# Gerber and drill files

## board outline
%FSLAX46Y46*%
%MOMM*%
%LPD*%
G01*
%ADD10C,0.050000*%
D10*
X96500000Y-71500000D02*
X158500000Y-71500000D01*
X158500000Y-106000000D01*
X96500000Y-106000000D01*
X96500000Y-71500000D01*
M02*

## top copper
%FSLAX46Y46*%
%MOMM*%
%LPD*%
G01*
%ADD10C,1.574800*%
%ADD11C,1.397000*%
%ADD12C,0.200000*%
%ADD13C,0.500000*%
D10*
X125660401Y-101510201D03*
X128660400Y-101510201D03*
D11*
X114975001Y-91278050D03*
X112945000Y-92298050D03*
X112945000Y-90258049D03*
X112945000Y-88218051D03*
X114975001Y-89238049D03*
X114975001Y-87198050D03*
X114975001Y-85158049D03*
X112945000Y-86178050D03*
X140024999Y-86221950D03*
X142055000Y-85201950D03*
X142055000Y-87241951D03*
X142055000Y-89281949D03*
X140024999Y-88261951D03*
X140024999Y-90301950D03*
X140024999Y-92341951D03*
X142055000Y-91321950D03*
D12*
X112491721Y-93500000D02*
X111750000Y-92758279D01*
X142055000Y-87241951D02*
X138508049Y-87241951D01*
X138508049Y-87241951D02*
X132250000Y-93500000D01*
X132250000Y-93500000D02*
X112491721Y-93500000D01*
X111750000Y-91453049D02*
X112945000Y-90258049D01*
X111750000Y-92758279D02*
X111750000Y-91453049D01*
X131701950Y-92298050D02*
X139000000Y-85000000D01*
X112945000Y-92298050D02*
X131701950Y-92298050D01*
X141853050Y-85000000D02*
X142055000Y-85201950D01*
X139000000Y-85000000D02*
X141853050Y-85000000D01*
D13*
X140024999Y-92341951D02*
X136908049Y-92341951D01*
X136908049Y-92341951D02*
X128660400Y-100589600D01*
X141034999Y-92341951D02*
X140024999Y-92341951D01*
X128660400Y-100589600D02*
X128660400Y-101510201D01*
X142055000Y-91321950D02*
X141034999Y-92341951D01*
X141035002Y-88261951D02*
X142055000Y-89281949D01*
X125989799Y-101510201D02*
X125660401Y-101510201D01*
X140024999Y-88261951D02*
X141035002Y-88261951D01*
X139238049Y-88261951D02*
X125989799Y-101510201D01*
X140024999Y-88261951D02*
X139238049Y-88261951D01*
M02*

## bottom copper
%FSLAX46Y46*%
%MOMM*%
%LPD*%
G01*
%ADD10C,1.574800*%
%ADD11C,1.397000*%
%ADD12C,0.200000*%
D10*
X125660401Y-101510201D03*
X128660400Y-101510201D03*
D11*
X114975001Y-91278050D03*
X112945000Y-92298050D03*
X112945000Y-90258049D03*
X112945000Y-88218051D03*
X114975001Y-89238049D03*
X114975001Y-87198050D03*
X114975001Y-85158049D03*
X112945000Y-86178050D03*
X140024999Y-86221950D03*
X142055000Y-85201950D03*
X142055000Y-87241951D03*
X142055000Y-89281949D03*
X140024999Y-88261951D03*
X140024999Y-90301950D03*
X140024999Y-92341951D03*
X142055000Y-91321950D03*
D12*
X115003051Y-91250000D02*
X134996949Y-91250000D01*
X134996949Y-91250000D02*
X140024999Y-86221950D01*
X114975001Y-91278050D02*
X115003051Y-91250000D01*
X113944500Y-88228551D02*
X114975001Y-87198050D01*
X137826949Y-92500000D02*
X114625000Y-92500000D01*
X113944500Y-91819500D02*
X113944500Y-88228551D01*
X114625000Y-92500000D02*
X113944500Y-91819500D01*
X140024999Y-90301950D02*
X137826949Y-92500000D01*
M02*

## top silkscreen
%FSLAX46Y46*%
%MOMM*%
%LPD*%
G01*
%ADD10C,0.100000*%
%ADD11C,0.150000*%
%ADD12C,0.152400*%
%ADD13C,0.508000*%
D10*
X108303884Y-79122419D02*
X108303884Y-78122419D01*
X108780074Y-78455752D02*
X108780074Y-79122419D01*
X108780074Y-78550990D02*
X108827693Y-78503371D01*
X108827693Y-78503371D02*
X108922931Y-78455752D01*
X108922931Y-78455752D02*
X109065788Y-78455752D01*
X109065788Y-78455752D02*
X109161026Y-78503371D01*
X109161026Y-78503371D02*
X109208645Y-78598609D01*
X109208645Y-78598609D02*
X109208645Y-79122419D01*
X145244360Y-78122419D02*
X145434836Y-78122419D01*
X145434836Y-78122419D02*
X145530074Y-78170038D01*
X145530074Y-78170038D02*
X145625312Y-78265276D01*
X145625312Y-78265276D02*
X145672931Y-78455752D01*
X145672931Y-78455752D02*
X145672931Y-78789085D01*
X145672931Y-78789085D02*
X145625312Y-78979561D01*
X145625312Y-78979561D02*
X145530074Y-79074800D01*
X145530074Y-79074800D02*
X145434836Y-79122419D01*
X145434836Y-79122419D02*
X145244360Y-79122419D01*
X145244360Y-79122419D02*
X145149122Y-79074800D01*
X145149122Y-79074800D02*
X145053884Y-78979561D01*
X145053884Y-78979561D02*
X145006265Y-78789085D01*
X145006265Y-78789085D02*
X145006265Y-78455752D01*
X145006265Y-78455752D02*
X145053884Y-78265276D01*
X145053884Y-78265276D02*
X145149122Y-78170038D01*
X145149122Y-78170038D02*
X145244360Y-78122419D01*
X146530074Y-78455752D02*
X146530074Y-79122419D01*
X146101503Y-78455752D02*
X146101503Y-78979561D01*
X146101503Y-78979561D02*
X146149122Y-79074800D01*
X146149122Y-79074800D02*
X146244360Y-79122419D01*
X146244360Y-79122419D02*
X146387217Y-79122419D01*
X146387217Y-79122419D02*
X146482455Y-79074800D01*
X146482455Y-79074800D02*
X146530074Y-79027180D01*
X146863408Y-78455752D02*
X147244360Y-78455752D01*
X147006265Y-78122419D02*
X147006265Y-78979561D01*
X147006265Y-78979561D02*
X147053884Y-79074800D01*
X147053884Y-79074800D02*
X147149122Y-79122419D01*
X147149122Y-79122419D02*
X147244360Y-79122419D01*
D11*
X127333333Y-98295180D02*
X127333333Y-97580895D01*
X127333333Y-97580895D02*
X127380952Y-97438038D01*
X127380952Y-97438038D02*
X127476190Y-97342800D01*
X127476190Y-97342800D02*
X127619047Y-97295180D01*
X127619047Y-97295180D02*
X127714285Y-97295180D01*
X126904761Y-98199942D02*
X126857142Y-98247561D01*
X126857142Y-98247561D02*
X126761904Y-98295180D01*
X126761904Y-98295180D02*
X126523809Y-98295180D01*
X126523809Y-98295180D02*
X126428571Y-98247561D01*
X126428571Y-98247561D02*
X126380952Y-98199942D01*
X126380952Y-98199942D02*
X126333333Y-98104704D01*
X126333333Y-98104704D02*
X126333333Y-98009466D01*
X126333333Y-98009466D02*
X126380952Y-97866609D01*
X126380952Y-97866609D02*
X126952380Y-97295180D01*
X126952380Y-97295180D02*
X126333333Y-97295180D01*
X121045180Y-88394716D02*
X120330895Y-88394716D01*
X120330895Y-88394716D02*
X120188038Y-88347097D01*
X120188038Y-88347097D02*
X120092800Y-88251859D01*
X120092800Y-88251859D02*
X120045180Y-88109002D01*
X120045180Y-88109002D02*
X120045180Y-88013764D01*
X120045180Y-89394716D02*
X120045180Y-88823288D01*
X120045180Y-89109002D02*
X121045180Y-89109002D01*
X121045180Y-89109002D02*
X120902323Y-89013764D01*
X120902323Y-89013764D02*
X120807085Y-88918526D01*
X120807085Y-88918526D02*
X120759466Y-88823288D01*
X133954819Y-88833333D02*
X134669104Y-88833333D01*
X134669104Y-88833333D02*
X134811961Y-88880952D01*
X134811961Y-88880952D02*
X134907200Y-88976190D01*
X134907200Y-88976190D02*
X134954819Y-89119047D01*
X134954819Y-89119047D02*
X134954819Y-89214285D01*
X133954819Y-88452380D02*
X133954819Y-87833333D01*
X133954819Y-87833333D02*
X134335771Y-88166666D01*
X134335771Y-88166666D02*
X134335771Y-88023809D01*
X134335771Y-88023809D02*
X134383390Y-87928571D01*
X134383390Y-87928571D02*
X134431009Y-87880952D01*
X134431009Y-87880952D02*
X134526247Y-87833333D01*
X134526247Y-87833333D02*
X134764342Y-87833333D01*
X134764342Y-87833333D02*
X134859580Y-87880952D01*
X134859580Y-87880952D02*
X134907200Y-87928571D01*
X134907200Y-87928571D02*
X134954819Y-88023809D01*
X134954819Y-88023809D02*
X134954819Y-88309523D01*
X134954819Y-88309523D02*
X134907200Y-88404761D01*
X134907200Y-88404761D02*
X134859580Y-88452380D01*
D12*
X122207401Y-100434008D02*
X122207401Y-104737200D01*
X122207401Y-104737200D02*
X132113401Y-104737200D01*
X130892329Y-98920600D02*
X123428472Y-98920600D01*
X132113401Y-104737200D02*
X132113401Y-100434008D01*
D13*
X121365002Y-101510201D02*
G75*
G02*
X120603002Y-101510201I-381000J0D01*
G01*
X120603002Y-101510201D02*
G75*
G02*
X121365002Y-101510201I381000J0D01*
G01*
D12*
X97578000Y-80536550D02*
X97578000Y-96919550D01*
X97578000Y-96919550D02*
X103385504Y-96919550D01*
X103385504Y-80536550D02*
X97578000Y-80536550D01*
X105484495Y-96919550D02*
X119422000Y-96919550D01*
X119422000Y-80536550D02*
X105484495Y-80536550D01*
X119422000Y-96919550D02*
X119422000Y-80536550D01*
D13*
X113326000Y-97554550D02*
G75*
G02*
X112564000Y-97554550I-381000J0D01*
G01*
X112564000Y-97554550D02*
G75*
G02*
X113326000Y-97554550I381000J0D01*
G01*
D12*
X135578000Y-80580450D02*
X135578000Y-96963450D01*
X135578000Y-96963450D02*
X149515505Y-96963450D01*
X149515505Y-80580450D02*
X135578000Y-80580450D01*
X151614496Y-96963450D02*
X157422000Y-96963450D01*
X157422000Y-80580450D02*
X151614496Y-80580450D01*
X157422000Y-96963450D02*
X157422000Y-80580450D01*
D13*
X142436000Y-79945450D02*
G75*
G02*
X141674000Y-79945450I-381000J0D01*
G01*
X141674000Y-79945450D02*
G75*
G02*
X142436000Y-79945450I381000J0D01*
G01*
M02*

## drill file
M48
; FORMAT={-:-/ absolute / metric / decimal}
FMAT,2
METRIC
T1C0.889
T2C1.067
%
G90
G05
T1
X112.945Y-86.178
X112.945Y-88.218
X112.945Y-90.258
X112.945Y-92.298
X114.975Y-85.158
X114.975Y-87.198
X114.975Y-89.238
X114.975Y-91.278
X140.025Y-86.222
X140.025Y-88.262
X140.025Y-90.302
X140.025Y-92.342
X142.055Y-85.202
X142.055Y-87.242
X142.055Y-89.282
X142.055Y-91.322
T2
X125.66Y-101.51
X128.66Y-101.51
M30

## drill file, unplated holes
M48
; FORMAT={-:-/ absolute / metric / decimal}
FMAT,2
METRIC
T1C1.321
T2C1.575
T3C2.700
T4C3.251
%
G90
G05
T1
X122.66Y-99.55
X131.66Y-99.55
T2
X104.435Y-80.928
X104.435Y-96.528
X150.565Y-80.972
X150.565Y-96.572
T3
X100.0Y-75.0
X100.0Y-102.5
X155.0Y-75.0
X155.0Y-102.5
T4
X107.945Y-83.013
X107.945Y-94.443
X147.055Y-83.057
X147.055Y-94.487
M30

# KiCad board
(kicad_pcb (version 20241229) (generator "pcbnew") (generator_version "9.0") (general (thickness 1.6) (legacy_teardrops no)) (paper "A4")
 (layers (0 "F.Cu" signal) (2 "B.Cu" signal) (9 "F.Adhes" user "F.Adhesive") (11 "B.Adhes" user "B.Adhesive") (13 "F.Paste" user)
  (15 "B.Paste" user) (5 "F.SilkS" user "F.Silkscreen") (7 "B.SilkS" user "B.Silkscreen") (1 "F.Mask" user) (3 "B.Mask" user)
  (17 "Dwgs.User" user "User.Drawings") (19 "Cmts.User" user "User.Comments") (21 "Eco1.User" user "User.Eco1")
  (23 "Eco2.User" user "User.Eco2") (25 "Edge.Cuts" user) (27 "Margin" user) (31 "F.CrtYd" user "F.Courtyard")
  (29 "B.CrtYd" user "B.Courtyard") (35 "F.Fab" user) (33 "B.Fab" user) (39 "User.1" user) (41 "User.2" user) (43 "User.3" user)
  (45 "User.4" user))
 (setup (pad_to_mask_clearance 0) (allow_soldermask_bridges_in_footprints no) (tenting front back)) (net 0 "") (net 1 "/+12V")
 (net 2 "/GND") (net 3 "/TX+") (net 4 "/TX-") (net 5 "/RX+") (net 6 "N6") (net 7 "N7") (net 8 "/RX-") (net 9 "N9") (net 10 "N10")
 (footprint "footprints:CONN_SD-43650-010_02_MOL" (layer "F.Cu") (at 125.660401 101.510201 180)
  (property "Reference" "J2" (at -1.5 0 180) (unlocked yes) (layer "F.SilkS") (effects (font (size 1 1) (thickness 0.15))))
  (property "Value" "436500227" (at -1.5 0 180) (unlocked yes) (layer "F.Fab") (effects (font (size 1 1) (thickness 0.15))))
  (fp_line (start 3.453 1.076193) (end 3.453 -3.226999) (stroke (width 0.1524) (type solid)) (layer "F.SilkS"))
  (fp_line (start 3.453 -3.226999) (end -6.453 -3.226999) (stroke (width 0.1524) (type solid)) (layer "F.SilkS"))
  (fp_line (start -5.231928 2.589601) (end 2.231929 2.589601) (stroke (width 0.1524) (type solid)) (layer "F.SilkS"))
  (fp_line (start -6.453 -3.226999) (end -6.453 1.076193) (stroke (width 0.1524) (type solid)) (layer "F.SilkS"))
  (fp_circle (center 4.676399 0) (end 5.057399 0) (stroke (width 0.508) (type solid)) (fill no) (layer "F.SilkS"))
  (pad "" np_thru_hole circle (at -5.999998 1.960001 180) (size 1.3208 1.3208) (drill 1.3208) (layers "*.Cu" "*.Mask"))
  (pad "" np_thru_hole circle (at 2.999999 1.960001 180) (size 1.3208 1.3208) (drill 1.3208) (layers "*.Cu" "*.Mask"))
  (pad "1" thru_hole circle (at 0 0 180) (size 1.5748 1.5748) (drill 1.0668) (layers "*.Cu" "*.Mask") (remove_unused_layers no)
   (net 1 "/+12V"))
  (pad "2" thru_hole circle (at -2.999999 0 180) (size 1.5748 1.5748) (drill 1.0668) (layers "*.Cu" "*.Mask") (remove_unused_layers no)
   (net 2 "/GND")))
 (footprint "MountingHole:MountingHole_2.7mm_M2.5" (layer "F.Cu") (at 155 102.5)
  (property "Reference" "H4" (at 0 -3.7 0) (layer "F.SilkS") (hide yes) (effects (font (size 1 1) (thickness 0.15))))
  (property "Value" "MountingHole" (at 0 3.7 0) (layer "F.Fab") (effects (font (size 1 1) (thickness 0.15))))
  (pad "" np_thru_hole circle (at 0 0) (size 2.7 2.7) (drill 2.7) (layers "*.Cu" "*.Mask")))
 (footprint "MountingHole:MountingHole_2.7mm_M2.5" (layer "F.Cu") (at 155 75)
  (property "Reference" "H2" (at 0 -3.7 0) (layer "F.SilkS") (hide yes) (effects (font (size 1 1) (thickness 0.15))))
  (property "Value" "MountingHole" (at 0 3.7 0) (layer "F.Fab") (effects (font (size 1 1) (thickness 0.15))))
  (pad "" np_thru_hole circle (at 0 0) (size 2.7 2.7) (drill 2.7) (layers "*.Cu" "*.Mask")))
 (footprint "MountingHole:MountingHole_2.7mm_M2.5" (layer "F.Cu") (at 100 75)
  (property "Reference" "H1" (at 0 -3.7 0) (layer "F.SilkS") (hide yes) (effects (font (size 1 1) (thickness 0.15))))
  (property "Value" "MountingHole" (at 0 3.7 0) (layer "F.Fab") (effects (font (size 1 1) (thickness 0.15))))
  (pad "" np_thru_hole circle (at 0 0) (size 2.7 2.7) (drill 2.7) (layers "*.Cu" "*.Mask")))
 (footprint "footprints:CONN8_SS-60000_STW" (layer "F.Cu") (at 112.945 92.29805 -90)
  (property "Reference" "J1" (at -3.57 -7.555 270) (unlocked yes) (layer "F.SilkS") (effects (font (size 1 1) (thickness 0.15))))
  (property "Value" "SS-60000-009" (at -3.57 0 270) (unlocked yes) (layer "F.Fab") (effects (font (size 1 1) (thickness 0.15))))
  (fp_line (start -11.7615 15.367) (end 4.6215 15.367) (stroke (width 0.1524) (type solid)) (layer "F.SilkS"))
  (fp_line (start 4.6215 15.367) (end 4.6215 9.559496) (stroke (width 0.1524) (type solid)) (layer "F.SilkS"))
  (fp_line (start -11.7615 9.559496) (end -11.7615 15.367) (stroke (width 0.1524) (type solid)) (layer "F.SilkS"))
  (fp_line (start 4.6215 7.460505) (end 4.6215 -6.477) (stroke (width 0.1524) (type solid)) (layer "F.SilkS"))
  (fp_line (start -11.7615 -6.477) (end -11.7615 7.460505) (stroke (width 0.1524) (type solid)) (layer "F.SilkS"))
  (fp_line (start 4.6215 -6.477) (end -11.7615 -6.477) (stroke (width 0.1524) (type solid)) (layer "F.SilkS"))
  (fp_circle (center 5.2565 0) (end 5.6375 0) (stroke (width 0.508) (type solid)) (fill no) (layer "F.SilkS"))
  (pad "" np_thru_hole circle (at -11.37 8.510001 270) (size 1.5748 1.5748) (drill 1.5748) (layers))
  (pad "" np_thru_hole circle (at -9.285 5 270) (size 3.2512 3.2512) (drill 3.2512) (layers "*.Cu" "*.Mask"))
  (pad "" np_thru_hole circle (at 2.145 5 270) (size 3.2512 3.2512) (drill 3.2512) (layers "*.Cu" "*.Mask"))
  (pad "" np_thru_hole circle (at 4.229999 8.510001 270) (size 1.5748 1.5748) (drill 1.5748) (layers))
  (pad "1" thru_hole circle (at -1.02 -2.030001 270) (size 1.397 1.397) (drill 0.889) (layers "*.Cu" "*.Mask") (remove_unused_layers no)
   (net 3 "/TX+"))
  (pad "2" thru_hole circle (at 0 0 270) (size 1.397 1.397) (drill 0.889) (layers "*.Cu" "*.Mask") (remove_unused_layers no) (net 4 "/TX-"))
  (pad "3" thru_hole circle (at -2.040001 0 270) (size 1.397 1.397) (drill 0.889) (layers "*.Cu" "*.Mask") (remove_unused_layers no)
   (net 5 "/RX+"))
  (pad "4" thru_hole circle (at -4.079999 0 270) (size 1.397 1.397) (drill 0.889) (layers "*.Cu" "*.Mask") (remove_unused_layers no)
   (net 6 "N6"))
  (pad "5" thru_hole circle (at -3.060001 -2.030001 270) (size 1.397 1.397) (drill 0.889) (layers "*.Cu" "*.Mask") (remove_unused_layers no)
   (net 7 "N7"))
  (pad "6" thru_hole circle (at -5.1 -2.030001 270) (size 1.397 1.397) (drill 0.889) (layers "*.Cu" "*.Mask") (remove_unused_layers no)
   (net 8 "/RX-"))
  (pad "7" thru_hole circle (at -7.140001 -2.030001 270) (size 1.397 1.397) (drill 0.889) (layers "*.Cu" "*.Mask") (remove_unused_layers no)
   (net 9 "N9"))
  (pad "8" thru_hole circle (at -6.12 0 270) (size 1.397 1.397) (drill 0.889) (layers "*.Cu" "*.Mask") (remove_unused_layers no)
   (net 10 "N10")))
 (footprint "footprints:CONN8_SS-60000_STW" (layer "F.Cu") (at 142.055 85.20195 90)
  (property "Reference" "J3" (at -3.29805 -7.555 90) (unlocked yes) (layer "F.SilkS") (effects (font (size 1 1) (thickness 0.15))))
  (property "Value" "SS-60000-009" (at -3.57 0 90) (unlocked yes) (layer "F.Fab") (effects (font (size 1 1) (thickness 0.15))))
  (fp_line (start 4.6215 -6.477) (end -11.7615 -6.477) (stroke (width 0.1524) (type solid)) (layer "F.SilkS"))
  (fp_line (start -11.7615 -6.477) (end -11.7615 7.460505) (stroke (width 0.1524) (type solid)) (layer "F.SilkS"))
  (fp_line (start 4.6215 7.460505) (end 4.6215 -6.477) (stroke (width 0.1524) (type solid)) (layer "F.SilkS"))
  (fp_line (start -11.7615 9.559496) (end -11.7615 15.367) (stroke (width 0.1524) (type solid)) (layer "F.SilkS"))
  (fp_line (start 4.6215 15.367) (end 4.6215 9.559496) (stroke (width 0.1524) (type solid)) (layer "F.SilkS"))
  (fp_line (start -11.7615 15.367) (end 4.6215 15.367) (stroke (width 0.1524) (type solid)) (layer "F.SilkS"))
  (fp_circle (center 5.2565 0) (end 5.6375 0) (stroke (width 0.508) (type solid)) (fill no) (layer "F.SilkS"))
  (pad "" np_thru_hole circle (at -11.37 8.510001 90) (size 1.5748 1.5748) (drill 1.5748) (layers))
  (pad "" np_thru_hole circle (at -9.285 5 90) (size 3.2512 3.2512) (drill 3.2512) (layers "*.Cu" "*.Mask"))
  (pad "" np_thru_hole circle (at 2.145 5 90) (size 3.2512 3.2512) (drill 3.2512) (layers "*.Cu" "*.Mask"))
  (pad "" np_thru_hole circle (at 4.229999 8.510001 90) (size 1.5748 1.5748) (drill 1.5748) (layers))
  (pad "1" thru_hole circle (at -1.02 -2.030001 90) (size 1.397 1.397) (drill 0.889) (layers "*.Cu" "*.Mask") (remove_unused_layers no)
   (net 3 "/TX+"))
  (pad "2" thru_hole circle (at 0 0 90) (size 1.397 1.397) (drill 0.889) (layers "*.Cu" "*.Mask") (remove_unused_layers no) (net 4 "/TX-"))
  (pad "3" thru_hole circle (at -2.040001 0 90) (size 1.397 1.397) (drill 0.889) (layers "*.Cu" "*.Mask") (remove_unused_layers no)
   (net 5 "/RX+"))
  (pad "4" thru_hole circle (at -4.079999 0 90) (size 1.397 1.397) (drill 0.889) (layers "*.Cu" "*.Mask") (remove_unused_layers no)
   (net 1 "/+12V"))
  (pad "5" thru_hole circle (at -3.060001 -2.030001 90) (size 1.397 1.397) (drill 0.889) (layers "*.Cu" "*.Mask") (remove_unused_layers no)
   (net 1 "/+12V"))
  (pad "6" thru_hole circle (at -5.1 -2.030001 90) (size 1.397 1.397) (drill 0.889) (layers "*.Cu" "*.Mask") (remove_unused_layers no)
   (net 8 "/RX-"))
  (pad "7" thru_hole circle (at -7.140001 -2.030001 90) (size 1.397 1.397) (drill 0.889) (layers "*.Cu" "*.Mask") (remove_unused_layers no)
   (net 2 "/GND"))
  (pad "8" thru_hole circle (at -6.12 0 90) (size 1.397 1.397) (drill 0.889) (layers "*.Cu" "*.Mask") (remove_unused_layers no)
   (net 2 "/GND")))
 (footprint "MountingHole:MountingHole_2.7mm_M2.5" (layer "F.Cu") (at 100 102.5)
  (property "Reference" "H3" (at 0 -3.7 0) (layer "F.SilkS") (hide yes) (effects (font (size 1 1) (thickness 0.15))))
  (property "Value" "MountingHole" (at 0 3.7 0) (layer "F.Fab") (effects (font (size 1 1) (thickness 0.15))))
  (pad "" np_thru_hole circle (at 0 0) (size 2.7 2.7) (drill 2.7) (layers "*.Cu" "*.Mask")))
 (gr_rect (start 96.5 71.5) (end 158.5 106) (stroke (width 0.05) (type default)) (fill no) (layer "Edge.Cuts"))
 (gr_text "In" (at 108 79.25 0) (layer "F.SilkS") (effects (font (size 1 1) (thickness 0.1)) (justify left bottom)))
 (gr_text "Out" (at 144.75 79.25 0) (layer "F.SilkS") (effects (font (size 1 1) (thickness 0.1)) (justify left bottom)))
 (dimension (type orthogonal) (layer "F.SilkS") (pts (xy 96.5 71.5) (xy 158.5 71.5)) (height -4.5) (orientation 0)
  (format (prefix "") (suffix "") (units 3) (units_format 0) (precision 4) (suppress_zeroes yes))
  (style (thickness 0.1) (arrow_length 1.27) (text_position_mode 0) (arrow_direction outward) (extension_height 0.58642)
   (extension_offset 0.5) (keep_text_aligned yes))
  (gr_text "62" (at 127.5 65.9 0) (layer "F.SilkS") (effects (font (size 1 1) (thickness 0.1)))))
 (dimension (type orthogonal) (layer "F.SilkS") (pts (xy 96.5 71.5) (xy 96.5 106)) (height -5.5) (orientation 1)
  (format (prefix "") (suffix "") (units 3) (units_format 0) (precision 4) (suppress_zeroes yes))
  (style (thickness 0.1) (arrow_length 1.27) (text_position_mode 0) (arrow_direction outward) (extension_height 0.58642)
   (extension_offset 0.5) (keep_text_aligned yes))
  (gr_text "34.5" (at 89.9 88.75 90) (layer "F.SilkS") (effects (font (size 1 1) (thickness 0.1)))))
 (segment (start 112.491721 93.5) (end 111.75 92.758279) (width 0.2) (layer "F.Cu") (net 5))
 (segment (start 142.055 87.241951) (end 138.508049 87.241951) (width 0.2) (layer "F.Cu") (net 5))
 (segment (start 138.508049 87.241951) (end 132.25 93.5) (width 0.2) (layer "F.Cu") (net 5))
 (segment (start 132.25 93.5) (end 112.491721 93.5) (width 0.2) (layer "F.Cu") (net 5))
 (segment (start 111.75 91.453049) (end 112.945 90.258049) (width 0.2) (layer "F.Cu") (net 5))
 (segment (start 111.75 92.758279) (end 111.75 91.453049) (width 0.2) (layer "F.Cu") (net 5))
 (segment (start 115.003051 91.25) (end 134.996949 91.25) (width 0.2) (layer "B.Cu") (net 3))
 (segment (start 134.996949 91.25) (end 140.024999 86.22195) (width 0.2) (layer "B.Cu") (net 3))
 (segment (start 114.975001 91.27805) (end 115.003051 91.25) (width 0.2) (layer "B.Cu") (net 3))
 (segment (start 113.9445 88.228551) (end 114.975001 87.19805) (width 0.2) (layer "B.Cu") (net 8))
 (segment (start 137.826949 92.5) (end 114.625 92.5) (width 0.2) (layer "B.Cu") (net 8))
 (segment (start 113.9445 91.8195) (end 113.9445 88.228551) (width 0.2) (layer "B.Cu") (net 8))
 (segment (start 114.625 92.5) (end 113.9445 91.8195) (width 0.2) (layer "B.Cu") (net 8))
 (segment (start 140.024999 90.30195) (end 137.826949 92.5) (width 0.2) (layer "B.Cu") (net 8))
 (segment (start 131.70195 92.29805) (end 139 85) (width 0.2) (layer "F.Cu") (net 4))
 (segment (start 112.945 92.29805) (end 131.70195 92.29805) (width 0.2) (layer "F.Cu") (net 4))
 (segment (start 141.85305 85) (end 142.055 85.20195) (width 0.2) (layer "F.Cu") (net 4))
 (segment (start 139 85) (end 141.85305 85) (width 0.2) (layer "F.Cu") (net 4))
 (segment (start 140.024999 92.341951) (end 136.908049 92.341951) (width 0.5) (layer "F.Cu") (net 2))
 (segment (start 136.908049 92.341951) (end 128.6604 100.5896) (width 0.5) (layer "F.Cu") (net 2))
 (segment (start 141.034999 92.341951) (end 140.024999 92.341951) (width 0.5) (layer "F.Cu") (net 2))
 (segment (start 128.6604 100.5896) (end 128.6604 101.510201) (width 0.5) (layer "F.Cu") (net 2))
 (segment (start 142.055 91.32195) (end 141.034999 92.341951) (width 0.5) (layer "F.Cu") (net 2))
 (segment (start 141.035002 88.261951) (end 142.055 89.281949) (width 0.5) (layer "F.Cu") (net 1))
 (segment (start 125.989799 101.510201) (end 125.660401 101.510201) (width 0.5) (layer "F.Cu") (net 1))
 (segment (start 140.024999 88.261951) (end 141.035002 88.261951) (width 0.5) (layer "F.Cu") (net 1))
 (segment (start 139.238049 88.261951) (end 125.989799 101.510201) (width 0.5) (layer "F.Cu") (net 1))
 (segment (start 140.024999 88.261951) (end 139.238049 88.261951) (width 0.5) (layer "F.Cu") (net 1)))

